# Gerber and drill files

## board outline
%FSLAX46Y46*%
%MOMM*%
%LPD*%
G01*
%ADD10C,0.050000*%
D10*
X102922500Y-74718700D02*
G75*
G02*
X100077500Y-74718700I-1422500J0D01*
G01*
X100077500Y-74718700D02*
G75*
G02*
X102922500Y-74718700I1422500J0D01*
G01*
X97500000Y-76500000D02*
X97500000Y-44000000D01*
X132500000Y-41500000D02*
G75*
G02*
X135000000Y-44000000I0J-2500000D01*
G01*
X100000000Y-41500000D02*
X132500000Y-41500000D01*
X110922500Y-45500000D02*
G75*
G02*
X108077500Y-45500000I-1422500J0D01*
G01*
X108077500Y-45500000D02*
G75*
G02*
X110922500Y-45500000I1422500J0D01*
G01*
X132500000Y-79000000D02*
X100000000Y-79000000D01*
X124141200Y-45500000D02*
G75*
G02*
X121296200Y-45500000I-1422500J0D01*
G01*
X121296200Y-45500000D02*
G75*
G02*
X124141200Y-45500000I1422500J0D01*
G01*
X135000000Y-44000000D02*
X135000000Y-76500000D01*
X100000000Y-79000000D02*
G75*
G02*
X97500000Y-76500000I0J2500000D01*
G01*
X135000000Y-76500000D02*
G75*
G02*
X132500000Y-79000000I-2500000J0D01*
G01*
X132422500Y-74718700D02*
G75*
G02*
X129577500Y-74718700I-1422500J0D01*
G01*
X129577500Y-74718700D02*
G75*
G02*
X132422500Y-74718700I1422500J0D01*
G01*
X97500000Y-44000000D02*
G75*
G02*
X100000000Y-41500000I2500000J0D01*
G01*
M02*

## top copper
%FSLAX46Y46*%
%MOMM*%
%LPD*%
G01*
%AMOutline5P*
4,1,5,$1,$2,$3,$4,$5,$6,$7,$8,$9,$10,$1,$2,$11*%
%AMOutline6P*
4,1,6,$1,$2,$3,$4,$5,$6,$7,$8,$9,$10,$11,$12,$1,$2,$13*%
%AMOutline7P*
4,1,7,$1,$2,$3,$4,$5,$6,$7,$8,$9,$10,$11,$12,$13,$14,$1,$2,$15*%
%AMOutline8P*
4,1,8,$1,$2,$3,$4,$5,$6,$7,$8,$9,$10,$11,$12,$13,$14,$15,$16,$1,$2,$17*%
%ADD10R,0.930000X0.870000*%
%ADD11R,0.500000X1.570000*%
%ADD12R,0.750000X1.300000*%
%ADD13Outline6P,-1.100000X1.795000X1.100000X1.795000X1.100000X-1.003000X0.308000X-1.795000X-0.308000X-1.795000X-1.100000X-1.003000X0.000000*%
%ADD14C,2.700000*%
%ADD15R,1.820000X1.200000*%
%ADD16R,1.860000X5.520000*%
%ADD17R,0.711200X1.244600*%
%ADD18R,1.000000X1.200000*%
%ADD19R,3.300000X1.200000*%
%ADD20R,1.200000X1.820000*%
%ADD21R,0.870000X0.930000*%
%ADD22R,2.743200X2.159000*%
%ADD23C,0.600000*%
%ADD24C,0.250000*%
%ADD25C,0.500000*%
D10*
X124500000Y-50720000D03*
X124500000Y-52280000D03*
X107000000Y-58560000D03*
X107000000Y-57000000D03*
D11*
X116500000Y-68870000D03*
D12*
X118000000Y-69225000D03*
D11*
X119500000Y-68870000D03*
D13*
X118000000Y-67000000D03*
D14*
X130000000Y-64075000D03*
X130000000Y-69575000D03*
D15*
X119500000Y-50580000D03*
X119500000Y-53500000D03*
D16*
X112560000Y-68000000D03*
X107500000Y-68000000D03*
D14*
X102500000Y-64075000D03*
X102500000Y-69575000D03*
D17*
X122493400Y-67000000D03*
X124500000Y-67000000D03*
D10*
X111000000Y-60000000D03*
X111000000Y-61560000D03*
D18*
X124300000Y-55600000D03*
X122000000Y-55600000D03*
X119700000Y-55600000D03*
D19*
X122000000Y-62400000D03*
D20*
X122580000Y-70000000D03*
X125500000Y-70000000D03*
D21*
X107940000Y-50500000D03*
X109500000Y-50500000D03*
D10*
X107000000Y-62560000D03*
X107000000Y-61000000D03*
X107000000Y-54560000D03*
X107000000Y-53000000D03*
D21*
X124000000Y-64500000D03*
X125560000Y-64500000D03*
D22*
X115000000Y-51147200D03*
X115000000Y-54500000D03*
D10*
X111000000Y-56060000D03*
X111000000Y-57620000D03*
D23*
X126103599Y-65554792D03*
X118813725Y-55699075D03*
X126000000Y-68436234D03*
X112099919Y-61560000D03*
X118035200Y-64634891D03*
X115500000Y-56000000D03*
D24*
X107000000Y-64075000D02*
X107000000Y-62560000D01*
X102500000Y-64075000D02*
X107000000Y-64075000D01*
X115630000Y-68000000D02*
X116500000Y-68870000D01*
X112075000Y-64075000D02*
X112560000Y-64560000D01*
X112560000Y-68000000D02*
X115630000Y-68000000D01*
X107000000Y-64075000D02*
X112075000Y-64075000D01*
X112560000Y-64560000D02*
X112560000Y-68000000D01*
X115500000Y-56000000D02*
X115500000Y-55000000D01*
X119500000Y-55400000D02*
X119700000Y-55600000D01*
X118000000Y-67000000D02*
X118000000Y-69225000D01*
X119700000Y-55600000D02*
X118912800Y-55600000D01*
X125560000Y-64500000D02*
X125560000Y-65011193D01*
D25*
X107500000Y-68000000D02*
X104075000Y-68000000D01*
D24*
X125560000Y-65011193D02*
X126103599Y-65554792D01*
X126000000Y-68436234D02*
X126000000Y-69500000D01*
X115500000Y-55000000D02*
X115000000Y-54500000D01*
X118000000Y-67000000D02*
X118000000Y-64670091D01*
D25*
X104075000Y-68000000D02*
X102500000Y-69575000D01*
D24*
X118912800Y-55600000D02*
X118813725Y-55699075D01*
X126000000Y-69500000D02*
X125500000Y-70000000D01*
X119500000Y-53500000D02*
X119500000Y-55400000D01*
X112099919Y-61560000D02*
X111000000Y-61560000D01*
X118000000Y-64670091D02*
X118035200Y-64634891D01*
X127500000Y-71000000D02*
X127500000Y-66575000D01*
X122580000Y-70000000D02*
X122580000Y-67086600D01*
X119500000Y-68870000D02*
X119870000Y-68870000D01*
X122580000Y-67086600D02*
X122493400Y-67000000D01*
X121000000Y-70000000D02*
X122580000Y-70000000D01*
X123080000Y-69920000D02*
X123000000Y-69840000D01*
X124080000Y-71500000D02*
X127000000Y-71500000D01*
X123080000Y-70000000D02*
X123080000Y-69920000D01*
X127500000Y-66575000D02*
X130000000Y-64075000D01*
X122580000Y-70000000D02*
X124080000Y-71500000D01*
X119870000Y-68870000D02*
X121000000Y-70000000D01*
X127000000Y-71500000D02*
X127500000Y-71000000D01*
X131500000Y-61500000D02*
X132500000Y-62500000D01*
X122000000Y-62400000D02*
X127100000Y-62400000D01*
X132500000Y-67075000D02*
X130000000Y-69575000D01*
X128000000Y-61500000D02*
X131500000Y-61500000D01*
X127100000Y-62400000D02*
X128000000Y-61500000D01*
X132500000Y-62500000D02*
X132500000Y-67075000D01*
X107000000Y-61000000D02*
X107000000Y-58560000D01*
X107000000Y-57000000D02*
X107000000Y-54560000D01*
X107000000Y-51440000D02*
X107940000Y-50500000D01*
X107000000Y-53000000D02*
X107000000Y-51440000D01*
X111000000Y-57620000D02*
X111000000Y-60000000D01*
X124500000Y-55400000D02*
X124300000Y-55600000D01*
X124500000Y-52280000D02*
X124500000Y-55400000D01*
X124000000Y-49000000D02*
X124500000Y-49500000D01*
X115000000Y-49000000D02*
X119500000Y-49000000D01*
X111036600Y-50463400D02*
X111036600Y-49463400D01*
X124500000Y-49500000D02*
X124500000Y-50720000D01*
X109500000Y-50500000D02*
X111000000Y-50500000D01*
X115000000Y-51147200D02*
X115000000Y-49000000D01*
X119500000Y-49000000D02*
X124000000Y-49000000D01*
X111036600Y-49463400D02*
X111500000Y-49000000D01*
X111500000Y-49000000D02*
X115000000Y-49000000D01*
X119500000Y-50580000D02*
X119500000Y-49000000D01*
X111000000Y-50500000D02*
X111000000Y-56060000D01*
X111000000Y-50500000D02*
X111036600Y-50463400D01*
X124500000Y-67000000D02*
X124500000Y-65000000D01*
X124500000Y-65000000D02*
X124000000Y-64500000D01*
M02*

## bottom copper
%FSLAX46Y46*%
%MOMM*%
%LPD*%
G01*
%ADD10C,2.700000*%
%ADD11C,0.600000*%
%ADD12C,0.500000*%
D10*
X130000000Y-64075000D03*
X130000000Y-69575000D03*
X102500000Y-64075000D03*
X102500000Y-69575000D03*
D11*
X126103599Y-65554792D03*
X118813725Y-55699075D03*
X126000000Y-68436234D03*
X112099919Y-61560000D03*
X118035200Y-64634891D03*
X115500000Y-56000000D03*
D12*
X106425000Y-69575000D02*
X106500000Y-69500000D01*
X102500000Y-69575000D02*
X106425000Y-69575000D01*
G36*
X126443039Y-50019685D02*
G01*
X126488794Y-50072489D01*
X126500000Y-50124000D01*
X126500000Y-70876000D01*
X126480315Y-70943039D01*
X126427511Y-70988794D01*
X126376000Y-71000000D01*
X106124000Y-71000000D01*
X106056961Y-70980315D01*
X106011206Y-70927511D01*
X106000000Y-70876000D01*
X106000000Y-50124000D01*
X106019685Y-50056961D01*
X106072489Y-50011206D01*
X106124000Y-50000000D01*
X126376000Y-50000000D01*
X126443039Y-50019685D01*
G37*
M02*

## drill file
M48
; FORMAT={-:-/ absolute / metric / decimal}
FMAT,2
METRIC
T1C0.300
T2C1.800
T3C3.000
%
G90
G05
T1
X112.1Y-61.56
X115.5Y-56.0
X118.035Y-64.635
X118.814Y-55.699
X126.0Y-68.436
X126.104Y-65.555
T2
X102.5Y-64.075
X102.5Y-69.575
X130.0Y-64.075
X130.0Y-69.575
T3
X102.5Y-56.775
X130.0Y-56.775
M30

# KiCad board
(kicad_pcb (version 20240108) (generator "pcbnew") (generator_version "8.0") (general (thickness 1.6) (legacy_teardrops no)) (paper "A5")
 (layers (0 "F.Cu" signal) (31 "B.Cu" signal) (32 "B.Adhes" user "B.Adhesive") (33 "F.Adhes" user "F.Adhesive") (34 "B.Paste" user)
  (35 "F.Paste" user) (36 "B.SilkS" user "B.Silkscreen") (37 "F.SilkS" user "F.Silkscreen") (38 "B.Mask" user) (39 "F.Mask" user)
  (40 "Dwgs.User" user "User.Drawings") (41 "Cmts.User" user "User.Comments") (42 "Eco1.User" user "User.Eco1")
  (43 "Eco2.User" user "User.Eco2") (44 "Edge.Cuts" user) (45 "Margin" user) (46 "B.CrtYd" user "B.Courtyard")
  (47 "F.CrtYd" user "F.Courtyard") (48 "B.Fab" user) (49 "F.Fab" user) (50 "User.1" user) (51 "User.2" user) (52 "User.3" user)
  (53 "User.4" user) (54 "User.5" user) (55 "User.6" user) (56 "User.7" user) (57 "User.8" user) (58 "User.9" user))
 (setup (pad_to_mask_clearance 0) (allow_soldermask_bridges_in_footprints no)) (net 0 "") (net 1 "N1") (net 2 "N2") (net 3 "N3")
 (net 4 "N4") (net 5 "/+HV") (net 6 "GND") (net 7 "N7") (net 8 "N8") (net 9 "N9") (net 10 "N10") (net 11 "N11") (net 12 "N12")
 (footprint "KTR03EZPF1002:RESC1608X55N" (layer "F.Cu") (at 124.5 51.5 -90)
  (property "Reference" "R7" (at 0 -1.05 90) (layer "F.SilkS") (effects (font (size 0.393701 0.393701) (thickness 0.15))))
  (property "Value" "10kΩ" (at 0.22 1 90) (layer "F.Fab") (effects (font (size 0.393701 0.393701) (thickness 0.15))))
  (pad "1" smd rect (at -0.78 0 270) (size 0.87 0.93) (layers "F.Cu" "F.Paste" "F.Mask") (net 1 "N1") (solder_mask_margin 0.102))
  (pad "2" smd rect (at 0.78 0 270) (size 0.87 0.93) (layers "F.Cu" "F.Paste" "F.Mask") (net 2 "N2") (solder_mask_margin 0.102)))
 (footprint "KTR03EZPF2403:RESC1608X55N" (layer "F.Cu") (at 107 57.78 90)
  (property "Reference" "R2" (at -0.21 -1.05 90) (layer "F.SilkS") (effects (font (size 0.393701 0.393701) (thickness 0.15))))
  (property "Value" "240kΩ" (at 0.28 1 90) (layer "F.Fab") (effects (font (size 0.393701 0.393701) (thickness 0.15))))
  (pad "1" smd rect (at -0.78 0 90) (size 0.87 0.93) (layers "F.Cu" "F.Paste" "F.Mask") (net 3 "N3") (solder_mask_margin 0.102))
  (pad "2" smd rect (at 0.78 0 90) (size 0.87 0.93) (layers "F.Cu" "F.Paste" "F.Mask") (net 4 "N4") (solder_mask_margin 0.102)))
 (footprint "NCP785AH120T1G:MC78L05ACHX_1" (layer "F.Cu") (at 118 68.595)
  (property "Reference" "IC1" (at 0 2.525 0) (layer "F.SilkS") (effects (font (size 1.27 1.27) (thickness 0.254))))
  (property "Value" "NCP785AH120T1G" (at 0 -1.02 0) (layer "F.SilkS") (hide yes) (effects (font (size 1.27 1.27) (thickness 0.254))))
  (pad "1" smd rect (at -1.5 0.275) (size 0.5 1.57) (layers "F.Cu" "F.Paste" "F.Mask") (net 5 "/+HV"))
  (pad "2" smd rect (at 0 0.63) (size 0.75 1.3) (layers "F.Cu" "F.Paste" "F.Mask") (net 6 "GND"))
  (pad "3" smd rect (at 1.5 0.275) (size 0.5 1.57) (layers "F.Cu" "F.Paste" "F.Mask") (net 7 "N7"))
  (pad "4" smd roundrect (at 0 -1.595) (size 2.2 3.59) (layers "F.Cu" "F.Paste" "F.Mask") (roundrect_rratio 0) (chamfer_ratio 0.36)
   (chamfer bottom_left bottom_right) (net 6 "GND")))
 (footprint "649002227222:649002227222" (layer "F.Cu") (at 130 56.575 180)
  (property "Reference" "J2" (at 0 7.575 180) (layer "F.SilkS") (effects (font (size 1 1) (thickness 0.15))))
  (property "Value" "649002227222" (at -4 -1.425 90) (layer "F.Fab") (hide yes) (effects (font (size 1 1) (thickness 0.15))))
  (pad "" np_thru_hole circle (at 0 -0.2 180) (size 3 3) (drill 3) (layers "*.Cu" "*.Mask"))
  (pad "1" thru_hole circle (at 0 -7.5 180) (size 2.7 2.7) (drill 1.8) (layers "*.Cu" "*.Mask") (remove_unused_layers no) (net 7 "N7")
   (solder_mask_margin 0.102))
  (pad "2" thru_hole circle (at 0 -13 180) (size 2.7 2.7) (drill 1.8) (layers "*.Cu" "*.Mask") (remove_unused_layers no) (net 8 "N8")
   (solder_mask_margin 0.102)))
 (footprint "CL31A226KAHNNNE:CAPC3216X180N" (layer "F.Cu") (at 119.5 52.04 -90)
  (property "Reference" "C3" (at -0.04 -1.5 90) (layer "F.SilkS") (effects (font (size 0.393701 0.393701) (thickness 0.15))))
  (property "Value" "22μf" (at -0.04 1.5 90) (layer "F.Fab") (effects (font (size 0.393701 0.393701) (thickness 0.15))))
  (pad "1" smd rect (at -1.46 0 270) (size 1.2 1.82) (layers "F.Cu" "F.Paste" "F.Mask") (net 1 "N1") (solder_mask_margin 0.102))
  (pad "2" smd rect (at 1.46 0 270) (size 1.2 1.82) (layers "F.Cu" "F.Paste" "F.Mask") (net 6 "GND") (solder_mask_margin 0.102)))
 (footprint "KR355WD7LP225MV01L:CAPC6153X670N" (layer "F.Cu") (at 110.03 68 180)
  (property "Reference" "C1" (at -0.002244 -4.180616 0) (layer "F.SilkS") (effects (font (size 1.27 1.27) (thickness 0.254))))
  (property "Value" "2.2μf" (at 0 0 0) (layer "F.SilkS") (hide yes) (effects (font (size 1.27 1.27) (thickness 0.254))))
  (pad "1" smd rect (at -2.53 0 180) (size 1.86 5.52) (layers "F.Cu" "F.Paste" "F.Mask") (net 5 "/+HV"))
  (pad "2" smd rect (at 2.53 0 180) (size 1.86 5.52) (layers "F.Cu" "F.Paste" "F.Mask") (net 6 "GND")))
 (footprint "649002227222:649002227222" (layer "F.Cu") (at 102.5 56.575 180)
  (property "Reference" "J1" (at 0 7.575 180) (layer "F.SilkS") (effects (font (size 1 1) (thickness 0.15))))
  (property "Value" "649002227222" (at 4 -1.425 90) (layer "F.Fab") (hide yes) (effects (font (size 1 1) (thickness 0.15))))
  (pad "" np_thru_hole circle (at 0 -0.2 180) (size 3 3) (drill 3) (layers "*.Cu" "*.Mask"))
  (pad "1" thru_hole circle (at 0 -7.5 180) (size 2.7 2.7) (drill 1.8) (layers "*.Cu" "*.Mask") (remove_unused_layers no) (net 5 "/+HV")
   (solder_mask_margin 0.102))
  (pad "2" thru_hole circle (at 0 -13 180) (size 2.7 2.7) (drill 1.8) (layers "*.Cu" "*.Mask") (remove_unused_layers no) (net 6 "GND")
   (solder_mask_margin 0.102)))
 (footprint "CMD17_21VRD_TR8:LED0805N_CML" (layer "F.Cu") (at 123.4967 67)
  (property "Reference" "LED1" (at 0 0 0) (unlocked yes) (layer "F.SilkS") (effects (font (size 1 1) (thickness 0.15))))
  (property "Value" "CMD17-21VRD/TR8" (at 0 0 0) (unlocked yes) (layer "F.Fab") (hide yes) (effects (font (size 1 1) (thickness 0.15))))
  (pad "1" smd rect (at -1.0033 0) (size 0.7112 1.2446) (layers "F.Cu" "F.Paste" "F.Mask") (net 7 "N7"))
  (pad "2" smd rect (at 1.0033 0) (size 0.7112 1.2446) (layers "F.Cu" "F.Paste" "F.Mask") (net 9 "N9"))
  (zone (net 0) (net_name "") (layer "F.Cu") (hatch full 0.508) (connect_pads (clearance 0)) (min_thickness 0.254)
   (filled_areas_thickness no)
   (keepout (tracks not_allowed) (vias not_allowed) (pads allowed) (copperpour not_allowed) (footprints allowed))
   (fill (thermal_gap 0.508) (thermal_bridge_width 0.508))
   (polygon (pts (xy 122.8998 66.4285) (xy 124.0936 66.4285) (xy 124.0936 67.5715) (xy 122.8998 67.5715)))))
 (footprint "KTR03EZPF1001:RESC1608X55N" (layer "F.Cu") (at 111 60.78 -90)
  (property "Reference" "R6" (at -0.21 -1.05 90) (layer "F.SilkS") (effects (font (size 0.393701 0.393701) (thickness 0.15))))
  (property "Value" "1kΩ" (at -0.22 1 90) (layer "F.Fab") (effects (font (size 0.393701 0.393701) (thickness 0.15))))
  (pad "1" smd rect (at -0.78 0 270) (size 0.87 0.93) (layers "F.Cu" "F.Paste" "F.Mask") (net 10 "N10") (solder_mask_margin 0.102))
  (pad "2" smd rect (at 0.78 0 270) (size 0.87 0.93) (layers "F.Cu" "F.Paste" "F.Mask") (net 6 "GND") (solder_mask_margin 0.102)))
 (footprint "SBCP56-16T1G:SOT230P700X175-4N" (layer "F.Cu") (at 122 59 -90)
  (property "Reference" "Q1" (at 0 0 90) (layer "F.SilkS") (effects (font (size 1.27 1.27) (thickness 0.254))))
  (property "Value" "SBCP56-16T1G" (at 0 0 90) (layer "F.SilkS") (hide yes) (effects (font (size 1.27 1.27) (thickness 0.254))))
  (pad "1" smd rect (at -3.4 -2.3) (size 1 1.2) (layers "F.Cu" "F.Paste" "F.Mask") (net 2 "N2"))
  (pad "2" smd rect (at -3.4 0) (size 1 1.2) (layers "F.Cu" "F.Paste" "F.Mask") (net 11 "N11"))
  (pad "3" smd rect (at -3.4 2.3) (size 1 1.2) (layers "F.Cu" "F.Paste" "F.Mask") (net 6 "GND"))
  (pad "4" smd rect (at 3.4 0 270) (size 1.2 3.3) (layers "F.Cu" "F.Paste" "F.Mask") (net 8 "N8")))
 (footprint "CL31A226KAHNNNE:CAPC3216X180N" (layer "F.Cu") (at 124.04 70)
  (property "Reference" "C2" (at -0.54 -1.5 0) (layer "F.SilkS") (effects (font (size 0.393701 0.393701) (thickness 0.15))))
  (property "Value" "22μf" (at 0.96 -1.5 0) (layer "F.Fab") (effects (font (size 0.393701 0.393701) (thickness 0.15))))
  (pad "1" smd rect (at -1.46 0) (size 1.2 1.82) (layers "F.Cu" "F.Paste" "F.Mask") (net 7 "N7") (solder_mask_margin 0.102))
  (pad "2" smd rect (at 1.46 0) (size 1.2 1.82) (layers "F.Cu" "F.Paste" "F.Mask") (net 6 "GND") (solder_mask_margin 0.102)))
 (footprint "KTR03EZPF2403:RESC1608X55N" (layer "F.Cu") (at 108.72 50.5)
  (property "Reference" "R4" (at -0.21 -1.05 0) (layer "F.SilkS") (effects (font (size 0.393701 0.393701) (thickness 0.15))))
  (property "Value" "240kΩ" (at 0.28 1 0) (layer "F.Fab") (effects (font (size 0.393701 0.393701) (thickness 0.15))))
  (pad "1" smd rect (at -0.78 0) (size 0.87 0.93) (layers "F.Cu" "F.Paste" "F.Mask") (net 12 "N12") (solder_mask_margin 0.102))
  (pad "2" smd rect (at 0.78 0) (size 0.87 0.93) (layers "F.Cu" "F.Paste" "F.Mask") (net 1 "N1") (solder_mask_margin 0.102)))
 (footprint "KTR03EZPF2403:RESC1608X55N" (layer "F.Cu") (at 107 61.78 90)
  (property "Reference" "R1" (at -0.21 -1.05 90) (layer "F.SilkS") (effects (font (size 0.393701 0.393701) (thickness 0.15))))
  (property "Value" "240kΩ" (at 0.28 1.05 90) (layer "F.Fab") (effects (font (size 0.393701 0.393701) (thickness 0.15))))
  (pad "1" smd rect (at -0.78 0 90) (size 0.87 0.93) (layers "F.Cu" "F.Paste" "F.Mask") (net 5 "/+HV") (solder_mask_margin 0.102))
  (pad "2" smd rect (at 0.78 0 90) (size 0.87 0.93) (layers "F.Cu" "F.Paste" "F.Mask") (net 3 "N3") (solder_mask_margin 0.102)))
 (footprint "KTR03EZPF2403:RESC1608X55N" (layer "F.Cu") (at 107 53.78 90)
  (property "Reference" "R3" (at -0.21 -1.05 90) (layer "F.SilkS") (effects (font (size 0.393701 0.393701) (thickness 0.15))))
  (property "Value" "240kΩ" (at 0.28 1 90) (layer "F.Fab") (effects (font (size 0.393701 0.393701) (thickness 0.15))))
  (pad "1" smd rect (at -0.78 0 90) (size 0.87 0.93) (layers "F.Cu" "F.Paste" "F.Mask") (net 4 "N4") (solder_mask_margin 0.102))
  (pad "2" smd rect (at 0.78 0 90) (size 0.87 0.93) (layers "F.Cu" "F.Paste" "F.Mask") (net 12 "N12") (solder_mask_margin 0.102)))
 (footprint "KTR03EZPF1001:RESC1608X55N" (layer "F.Cu") (at 124.78 64.5)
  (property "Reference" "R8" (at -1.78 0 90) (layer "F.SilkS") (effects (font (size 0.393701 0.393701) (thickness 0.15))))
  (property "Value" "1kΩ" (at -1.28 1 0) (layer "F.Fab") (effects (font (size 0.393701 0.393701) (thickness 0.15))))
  (pad "1" smd rect (at -0.78 0) (size 0.87 0.93) (layers "F.Cu" "F.Paste" "F.Mask") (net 9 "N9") (solder_mask_margin 0.102))
  (pad "2" smd rect (at 0.78 0) (size 0.87 0.93) (layers "F.Cu" "F.Paste" "F.Mask") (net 6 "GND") (solder_mask_margin 0.102)))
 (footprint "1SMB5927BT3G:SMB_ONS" (layer "F.Cu") (at 115 52.8236 -90)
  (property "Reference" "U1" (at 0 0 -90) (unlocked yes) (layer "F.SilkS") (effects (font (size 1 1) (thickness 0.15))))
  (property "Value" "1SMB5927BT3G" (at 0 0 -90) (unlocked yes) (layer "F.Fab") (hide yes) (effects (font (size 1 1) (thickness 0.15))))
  (pad "1" smd rect (at -1.6764 0 270) (size 2.159 2.7432) (layers "F.Cu" "F.Paste" "F.Mask") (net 1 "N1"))
  (pad "2" smd rect (at 1.6764 0 270) (size 2.159 2.7432) (layers "F.Cu" "F.Paste" "F.Mask") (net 6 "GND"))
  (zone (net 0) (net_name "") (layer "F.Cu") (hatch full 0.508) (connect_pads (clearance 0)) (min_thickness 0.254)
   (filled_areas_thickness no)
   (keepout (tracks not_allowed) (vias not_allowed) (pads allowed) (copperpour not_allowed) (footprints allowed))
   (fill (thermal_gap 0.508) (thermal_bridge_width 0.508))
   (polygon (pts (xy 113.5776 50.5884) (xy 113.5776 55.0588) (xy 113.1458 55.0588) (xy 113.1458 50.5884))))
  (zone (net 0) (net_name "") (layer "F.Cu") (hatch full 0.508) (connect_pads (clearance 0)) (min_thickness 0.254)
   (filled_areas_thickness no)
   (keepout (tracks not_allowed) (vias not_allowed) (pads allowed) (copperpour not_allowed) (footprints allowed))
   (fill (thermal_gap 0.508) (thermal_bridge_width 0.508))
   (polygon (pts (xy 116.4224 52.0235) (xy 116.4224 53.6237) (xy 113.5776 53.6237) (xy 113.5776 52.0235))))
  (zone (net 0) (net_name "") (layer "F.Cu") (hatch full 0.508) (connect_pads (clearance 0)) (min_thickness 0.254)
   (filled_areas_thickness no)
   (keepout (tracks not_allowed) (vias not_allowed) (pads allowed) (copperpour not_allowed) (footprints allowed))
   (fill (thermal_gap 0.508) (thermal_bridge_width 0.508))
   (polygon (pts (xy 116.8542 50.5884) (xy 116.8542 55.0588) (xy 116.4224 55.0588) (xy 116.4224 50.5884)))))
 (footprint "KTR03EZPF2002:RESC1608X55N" (layer "F.Cu") (at 111 56.84 -90)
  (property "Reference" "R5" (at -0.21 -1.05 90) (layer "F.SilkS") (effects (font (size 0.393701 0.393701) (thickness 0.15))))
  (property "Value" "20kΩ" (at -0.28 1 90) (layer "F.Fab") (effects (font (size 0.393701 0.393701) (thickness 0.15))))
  (pad "1" smd rect (at -0.78 0 270) (size 0.87 0.93) (layers "F.Cu" "F.Paste" "F.Mask") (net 1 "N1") (solder_mask_margin 0.102))
  (pad "2" smd rect (at 0.78 0 270) (size 0.87 0.93) (layers "F.Cu" "F.Paste" "F.Mask") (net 10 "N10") (solder_mask_margin 0.102)))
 (gr_circle (center 101.5 74.7187) (end 102.9225 74.7187) (stroke (width 0.05) (type default)) (fill none) (layer "Edge.Cuts"))
 (gr_line (start 97.5 76.5) (end 97.5 44) (stroke (width 0.05) (type default)) (layer "Edge.Cuts"))
 (gr_arc (start 132.5 41.5) (mid 134.267767 42.232233) (end 135 44) (stroke (width 0.05) (type default)) (layer "Edge.Cuts"))
 (gr_line (start 100 41.5) (end 132.5 41.5) (stroke (width 0.05) (type default)) (layer "Edge.Cuts"))
 (gr_circle (center 109.5 45.5) (end 110.9225 45.5) (stroke (width 0.05) (type default)) (fill none) (layer "Edge.Cuts"))
 (gr_line (start 132.5 79) (end 100 79) (stroke (width 0.05) (type default)) (layer "Edge.Cuts"))
 (gr_circle (center 122.7187 45.5) (end 124.1412 45.5) (stroke (width 0.05) (type default)) (fill none) (layer "Edge.Cuts"))
 (gr_line (start 135 44) (end 135 76.5) (stroke (width 0.05) (type default)) (layer "Edge.Cuts"))
 (gr_arc (start 100 79) (mid 98.232233 78.267767) (end 97.5 76.5) (stroke (width 0.05) (type default)) (layer "Edge.Cuts"))
 (gr_arc (start 135 76.5) (mid 134.267767 78.267767) (end 132.5 79) (stroke (width 0.05) (type default)) (layer "Edge.Cuts"))
 (gr_circle (center 131 74.7187) (end 132.4225 74.7187) (stroke (width 0.05) (type default)) (fill none) (layer "Edge.Cuts"))
 (gr_arc (start 97.5 44) (mid 98.232233 42.232233) (end 100 41.5) (stroke (width 0.05) (type default)) (layer "Edge.Cuts"))
 (segment (start 107 64.075) (end 107 62.56) (width 0.25) (layer "F.Cu") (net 5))
 (segment (start 102.5 64.075) (end 107 64.075) (width 0.25) (layer "F.Cu") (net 5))
 (segment (start 115.63 68) (end 116.5 68.87) (width 0.25) (layer "F.Cu") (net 5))
 (segment (start 112.075 64.075) (end 112.56 64.56) (width 0.25) (layer "F.Cu") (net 5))
 (segment (start 112.56 68) (end 115.63 68) (width 0.25) (layer "F.Cu") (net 5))
 (segment (start 107 64.075) (end 112.075 64.075) (width 0.25) (layer "F.Cu") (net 5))
 (segment (start 112.56 64.56) (end 112.56 68) (width 0.25) (layer "F.Cu") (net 5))
 (segment (start 115.5 56) (end 115.5 55) (width 0.25) (layer "F.Cu") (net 6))
 (segment (start 119.5 55.4) (end 119.7 55.6) (width 0.25) (layer "F.Cu") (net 6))
 (segment (start 118 67) (end 118 69.225) (width 0.25) (layer "F.Cu") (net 6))
 (segment (start 119.7 55.6) (end 118.9128 55.6) (width 0.25) (layer "F.Cu") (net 6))
 (segment (start 125.56 64.5) (end 125.56 65.011193) (width 0.25) (layer "F.Cu") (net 6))
 (segment (start 107.5 68) (end 104.075 68) (width 0.5) (layer "F.Cu") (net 6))
 (segment (start 125.56 65.011193) (end 126.103599 65.554792) (width 0.25) (layer "F.Cu") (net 6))
 (segment (start 126 68.436234) (end 126 69.5) (width 0.25) (layer "F.Cu") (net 6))
 (segment (start 115.5 55) (end 115 54.5) (width 0.25) (layer "F.Cu") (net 6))
 (segment (start 118 67) (end 118 64.670091) (width 0.25) (layer "F.Cu") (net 6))
 (segment (start 104.075 68) (end 102.5 69.575) (width 0.5) (layer "F.Cu") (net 6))
 (segment (start 118.9128 55.6) (end 118.813725 55.699075) (width 0.25) (layer "F.Cu") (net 6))
 (segment (start 126 69.5) (end 125.5 70) (width 0.25) (layer "F.Cu") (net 6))
 (segment (start 119.5 53.5) (end 119.5 55.4) (width 0.25) (layer "F.Cu") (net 6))
 (segment (start 112.099919 61.56) (end 111 61.56) (width 0.25) (layer "F.Cu") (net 6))
 (segment (start 118 64.670091) (end 118.0352 64.634891) (width 0.25) (layer "F.Cu") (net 6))
 (via (at 126.103599 65.554792) (size 0.6) (drill 0.3) (layers "F.Cu" "B.Cu") (free yes) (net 6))
 (via (at 118.813725 55.699075) (size 0.6) (drill 0.3) (layers "F.Cu" "B.Cu") (free yes) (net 6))
 (via (at 126 68.436234) (size 0.6) (drill 0.3) (layers "F.Cu" "B.Cu") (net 6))
 (via (at 112.099919 61.56) (size 0.6) (drill 0.3) (layers "F.Cu" "B.Cu") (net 6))
 (via (at 118.0352 64.634891) (size 0.6) (drill 0.3) (layers "F.Cu" "B.Cu") (free yes) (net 6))
 (via (at 115.5 56) (size 0.6) (drill 0.3) (layers "F.Cu" "B.Cu") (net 6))
 (segment (start 106.425 69.575) (end 106.5 69.5) (width 0.5) (layer "B.Cu") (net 6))
 (segment (start 102.5 69.575) (end 106.425 69.575) (width 0.5) (layer "B.Cu") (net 6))
 (segment (start 127.5 71) (end 127.5 66.575) (width 0.25) (layer "F.Cu") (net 7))
 (segment (start 122.58 70) (end 122.58 67.0866) (width 0.25) (layer "F.Cu") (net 7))
 (segment (start 119.5 68.87) (end 119.87 68.87) (width 0.25) (layer "F.Cu") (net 7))
 (segment (start 122.58 67.0866) (end 122.4934 67) (width 0.25) (layer "F.Cu") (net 7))
 (segment (start 121 70) (end 122.58 70) (width 0.25) (layer "F.Cu") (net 7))
 (segment (start 123.08 69.92) (end 123 69.84) (width 0.25) (layer "F.Cu") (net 7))
 (segment (start 124.08 71.5) (end 127 71.5) (width 0.25) (layer "F.Cu") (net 7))
 (segment (start 123.08 70) (end 123.08 69.92) (width 0.25) (layer "F.Cu") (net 7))
 (segment (start 127.5 66.575) (end 130 64.075) (width 0.25) (layer "F.Cu") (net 7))
 (segment (start 122.58 70) (end 124.08 71.5) (width 0.25) (layer "F.Cu") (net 7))
 (segment (start 119.87 68.87) (end 121 70) (width 0.25) (layer "F.Cu") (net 7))
 (segment (start 127 71.5) (end 127.5 71) (width 0.25) (layer "F.Cu") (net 7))
 (segment (start 131.5 61.5) (end 132.5 62.5) (width 0.25) (layer "F.Cu") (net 8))
 (segment (start 122 62.4) (end 127.1 62.4) (width 0.25) (layer "F.Cu") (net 8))
 (segment (start 132.5 67.075) (end 130 69.575) (width 0.25) (layer "F.Cu") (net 8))
 (segment (start 128 61.5) (end 131.5 61.5) (width 0.25) (layer "F.Cu") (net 8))
 (segment (start 127.1 62.4) (end 128 61.5) (width 0.25) (layer "F.Cu") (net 8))
 (segment (start 132.5 62.5) (end 132.5 67.075) (width 0.25) (layer "F.Cu") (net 8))
 (segment (start 107 61) (end 107 58.56) (width 0.25) (layer "F.Cu") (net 3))
 (segment (start 107 57) (end 107 54.56) (width 0.25) (layer "F.Cu") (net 4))
 (segment (start 107 51.44) (end 107.94 50.5) (width 0.25) (layer "F.Cu") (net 12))
 (segment (start 107 53) (end 107 51.44) (width 0.25) (layer "F.Cu") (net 12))
 (segment (start 111 57.62) (end 111 60) (width 0.25) (layer "F.Cu") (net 10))
 (segment (start 124.5 55.4) (end 124.3 55.6) (width 0.25) (layer "F.Cu") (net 2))
 (segment (start 124.5 52.28) (end 124.5 55.4) (width 0.25) (layer "F.Cu") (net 2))
 (segment (start 124 49) (end 124.5 49.5) (width 0.25) (layer "F.Cu") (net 1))
 (segment (start 115 49) (end 119.5 49) (width 0.25) (layer "F.Cu") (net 1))
 (segment (start 111.0366 50.4634) (end 111.0366 49.4634) (width 0.25) (layer "F.Cu") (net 1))
 (segment (start 124.5 49.5) (end 124.5 50.72) (width 0.25) (layer "F.Cu") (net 1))
 (segment (start 109.5 50.5) (end 111 50.5) (width 0.25) (layer "F.Cu") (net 1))
 (segment (start 115 51.1472) (end 115 49) (width 0.25) (layer "F.Cu") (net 1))
 (segment (start 119.5 49) (end 124 49) (width 0.25) (layer "F.Cu") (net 1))
 (segment (start 111.0366 49.4634) (end 111.5 49) (width 0.25) (layer "F.Cu") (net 1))
 (segment (start 111.5 49) (end 115 49) (width 0.25) (layer "F.Cu") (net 1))
 (segment (start 119.5 50.58) (end 119.5 49) (width 0.25) (layer "F.Cu") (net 1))
 (segment (start 111 50.5) (end 111 56.06) (width 0.25) (layer "F.Cu") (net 1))
 (segment (start 111 50.5) (end 111.0366 50.4634) (width 0.25) (layer "F.Cu") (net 1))
 (segment (start 124.5 67) (end 124.5 65) (width 0.25) (layer "F.Cu") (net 9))
 (segment (start 124.5 65) (end 124 64.5) (width 0.25) (layer "F.Cu") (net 9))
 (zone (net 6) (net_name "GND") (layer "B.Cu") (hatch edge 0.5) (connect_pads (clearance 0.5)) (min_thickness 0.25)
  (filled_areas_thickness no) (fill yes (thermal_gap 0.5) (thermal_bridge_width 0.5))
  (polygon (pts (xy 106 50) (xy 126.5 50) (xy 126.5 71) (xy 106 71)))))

